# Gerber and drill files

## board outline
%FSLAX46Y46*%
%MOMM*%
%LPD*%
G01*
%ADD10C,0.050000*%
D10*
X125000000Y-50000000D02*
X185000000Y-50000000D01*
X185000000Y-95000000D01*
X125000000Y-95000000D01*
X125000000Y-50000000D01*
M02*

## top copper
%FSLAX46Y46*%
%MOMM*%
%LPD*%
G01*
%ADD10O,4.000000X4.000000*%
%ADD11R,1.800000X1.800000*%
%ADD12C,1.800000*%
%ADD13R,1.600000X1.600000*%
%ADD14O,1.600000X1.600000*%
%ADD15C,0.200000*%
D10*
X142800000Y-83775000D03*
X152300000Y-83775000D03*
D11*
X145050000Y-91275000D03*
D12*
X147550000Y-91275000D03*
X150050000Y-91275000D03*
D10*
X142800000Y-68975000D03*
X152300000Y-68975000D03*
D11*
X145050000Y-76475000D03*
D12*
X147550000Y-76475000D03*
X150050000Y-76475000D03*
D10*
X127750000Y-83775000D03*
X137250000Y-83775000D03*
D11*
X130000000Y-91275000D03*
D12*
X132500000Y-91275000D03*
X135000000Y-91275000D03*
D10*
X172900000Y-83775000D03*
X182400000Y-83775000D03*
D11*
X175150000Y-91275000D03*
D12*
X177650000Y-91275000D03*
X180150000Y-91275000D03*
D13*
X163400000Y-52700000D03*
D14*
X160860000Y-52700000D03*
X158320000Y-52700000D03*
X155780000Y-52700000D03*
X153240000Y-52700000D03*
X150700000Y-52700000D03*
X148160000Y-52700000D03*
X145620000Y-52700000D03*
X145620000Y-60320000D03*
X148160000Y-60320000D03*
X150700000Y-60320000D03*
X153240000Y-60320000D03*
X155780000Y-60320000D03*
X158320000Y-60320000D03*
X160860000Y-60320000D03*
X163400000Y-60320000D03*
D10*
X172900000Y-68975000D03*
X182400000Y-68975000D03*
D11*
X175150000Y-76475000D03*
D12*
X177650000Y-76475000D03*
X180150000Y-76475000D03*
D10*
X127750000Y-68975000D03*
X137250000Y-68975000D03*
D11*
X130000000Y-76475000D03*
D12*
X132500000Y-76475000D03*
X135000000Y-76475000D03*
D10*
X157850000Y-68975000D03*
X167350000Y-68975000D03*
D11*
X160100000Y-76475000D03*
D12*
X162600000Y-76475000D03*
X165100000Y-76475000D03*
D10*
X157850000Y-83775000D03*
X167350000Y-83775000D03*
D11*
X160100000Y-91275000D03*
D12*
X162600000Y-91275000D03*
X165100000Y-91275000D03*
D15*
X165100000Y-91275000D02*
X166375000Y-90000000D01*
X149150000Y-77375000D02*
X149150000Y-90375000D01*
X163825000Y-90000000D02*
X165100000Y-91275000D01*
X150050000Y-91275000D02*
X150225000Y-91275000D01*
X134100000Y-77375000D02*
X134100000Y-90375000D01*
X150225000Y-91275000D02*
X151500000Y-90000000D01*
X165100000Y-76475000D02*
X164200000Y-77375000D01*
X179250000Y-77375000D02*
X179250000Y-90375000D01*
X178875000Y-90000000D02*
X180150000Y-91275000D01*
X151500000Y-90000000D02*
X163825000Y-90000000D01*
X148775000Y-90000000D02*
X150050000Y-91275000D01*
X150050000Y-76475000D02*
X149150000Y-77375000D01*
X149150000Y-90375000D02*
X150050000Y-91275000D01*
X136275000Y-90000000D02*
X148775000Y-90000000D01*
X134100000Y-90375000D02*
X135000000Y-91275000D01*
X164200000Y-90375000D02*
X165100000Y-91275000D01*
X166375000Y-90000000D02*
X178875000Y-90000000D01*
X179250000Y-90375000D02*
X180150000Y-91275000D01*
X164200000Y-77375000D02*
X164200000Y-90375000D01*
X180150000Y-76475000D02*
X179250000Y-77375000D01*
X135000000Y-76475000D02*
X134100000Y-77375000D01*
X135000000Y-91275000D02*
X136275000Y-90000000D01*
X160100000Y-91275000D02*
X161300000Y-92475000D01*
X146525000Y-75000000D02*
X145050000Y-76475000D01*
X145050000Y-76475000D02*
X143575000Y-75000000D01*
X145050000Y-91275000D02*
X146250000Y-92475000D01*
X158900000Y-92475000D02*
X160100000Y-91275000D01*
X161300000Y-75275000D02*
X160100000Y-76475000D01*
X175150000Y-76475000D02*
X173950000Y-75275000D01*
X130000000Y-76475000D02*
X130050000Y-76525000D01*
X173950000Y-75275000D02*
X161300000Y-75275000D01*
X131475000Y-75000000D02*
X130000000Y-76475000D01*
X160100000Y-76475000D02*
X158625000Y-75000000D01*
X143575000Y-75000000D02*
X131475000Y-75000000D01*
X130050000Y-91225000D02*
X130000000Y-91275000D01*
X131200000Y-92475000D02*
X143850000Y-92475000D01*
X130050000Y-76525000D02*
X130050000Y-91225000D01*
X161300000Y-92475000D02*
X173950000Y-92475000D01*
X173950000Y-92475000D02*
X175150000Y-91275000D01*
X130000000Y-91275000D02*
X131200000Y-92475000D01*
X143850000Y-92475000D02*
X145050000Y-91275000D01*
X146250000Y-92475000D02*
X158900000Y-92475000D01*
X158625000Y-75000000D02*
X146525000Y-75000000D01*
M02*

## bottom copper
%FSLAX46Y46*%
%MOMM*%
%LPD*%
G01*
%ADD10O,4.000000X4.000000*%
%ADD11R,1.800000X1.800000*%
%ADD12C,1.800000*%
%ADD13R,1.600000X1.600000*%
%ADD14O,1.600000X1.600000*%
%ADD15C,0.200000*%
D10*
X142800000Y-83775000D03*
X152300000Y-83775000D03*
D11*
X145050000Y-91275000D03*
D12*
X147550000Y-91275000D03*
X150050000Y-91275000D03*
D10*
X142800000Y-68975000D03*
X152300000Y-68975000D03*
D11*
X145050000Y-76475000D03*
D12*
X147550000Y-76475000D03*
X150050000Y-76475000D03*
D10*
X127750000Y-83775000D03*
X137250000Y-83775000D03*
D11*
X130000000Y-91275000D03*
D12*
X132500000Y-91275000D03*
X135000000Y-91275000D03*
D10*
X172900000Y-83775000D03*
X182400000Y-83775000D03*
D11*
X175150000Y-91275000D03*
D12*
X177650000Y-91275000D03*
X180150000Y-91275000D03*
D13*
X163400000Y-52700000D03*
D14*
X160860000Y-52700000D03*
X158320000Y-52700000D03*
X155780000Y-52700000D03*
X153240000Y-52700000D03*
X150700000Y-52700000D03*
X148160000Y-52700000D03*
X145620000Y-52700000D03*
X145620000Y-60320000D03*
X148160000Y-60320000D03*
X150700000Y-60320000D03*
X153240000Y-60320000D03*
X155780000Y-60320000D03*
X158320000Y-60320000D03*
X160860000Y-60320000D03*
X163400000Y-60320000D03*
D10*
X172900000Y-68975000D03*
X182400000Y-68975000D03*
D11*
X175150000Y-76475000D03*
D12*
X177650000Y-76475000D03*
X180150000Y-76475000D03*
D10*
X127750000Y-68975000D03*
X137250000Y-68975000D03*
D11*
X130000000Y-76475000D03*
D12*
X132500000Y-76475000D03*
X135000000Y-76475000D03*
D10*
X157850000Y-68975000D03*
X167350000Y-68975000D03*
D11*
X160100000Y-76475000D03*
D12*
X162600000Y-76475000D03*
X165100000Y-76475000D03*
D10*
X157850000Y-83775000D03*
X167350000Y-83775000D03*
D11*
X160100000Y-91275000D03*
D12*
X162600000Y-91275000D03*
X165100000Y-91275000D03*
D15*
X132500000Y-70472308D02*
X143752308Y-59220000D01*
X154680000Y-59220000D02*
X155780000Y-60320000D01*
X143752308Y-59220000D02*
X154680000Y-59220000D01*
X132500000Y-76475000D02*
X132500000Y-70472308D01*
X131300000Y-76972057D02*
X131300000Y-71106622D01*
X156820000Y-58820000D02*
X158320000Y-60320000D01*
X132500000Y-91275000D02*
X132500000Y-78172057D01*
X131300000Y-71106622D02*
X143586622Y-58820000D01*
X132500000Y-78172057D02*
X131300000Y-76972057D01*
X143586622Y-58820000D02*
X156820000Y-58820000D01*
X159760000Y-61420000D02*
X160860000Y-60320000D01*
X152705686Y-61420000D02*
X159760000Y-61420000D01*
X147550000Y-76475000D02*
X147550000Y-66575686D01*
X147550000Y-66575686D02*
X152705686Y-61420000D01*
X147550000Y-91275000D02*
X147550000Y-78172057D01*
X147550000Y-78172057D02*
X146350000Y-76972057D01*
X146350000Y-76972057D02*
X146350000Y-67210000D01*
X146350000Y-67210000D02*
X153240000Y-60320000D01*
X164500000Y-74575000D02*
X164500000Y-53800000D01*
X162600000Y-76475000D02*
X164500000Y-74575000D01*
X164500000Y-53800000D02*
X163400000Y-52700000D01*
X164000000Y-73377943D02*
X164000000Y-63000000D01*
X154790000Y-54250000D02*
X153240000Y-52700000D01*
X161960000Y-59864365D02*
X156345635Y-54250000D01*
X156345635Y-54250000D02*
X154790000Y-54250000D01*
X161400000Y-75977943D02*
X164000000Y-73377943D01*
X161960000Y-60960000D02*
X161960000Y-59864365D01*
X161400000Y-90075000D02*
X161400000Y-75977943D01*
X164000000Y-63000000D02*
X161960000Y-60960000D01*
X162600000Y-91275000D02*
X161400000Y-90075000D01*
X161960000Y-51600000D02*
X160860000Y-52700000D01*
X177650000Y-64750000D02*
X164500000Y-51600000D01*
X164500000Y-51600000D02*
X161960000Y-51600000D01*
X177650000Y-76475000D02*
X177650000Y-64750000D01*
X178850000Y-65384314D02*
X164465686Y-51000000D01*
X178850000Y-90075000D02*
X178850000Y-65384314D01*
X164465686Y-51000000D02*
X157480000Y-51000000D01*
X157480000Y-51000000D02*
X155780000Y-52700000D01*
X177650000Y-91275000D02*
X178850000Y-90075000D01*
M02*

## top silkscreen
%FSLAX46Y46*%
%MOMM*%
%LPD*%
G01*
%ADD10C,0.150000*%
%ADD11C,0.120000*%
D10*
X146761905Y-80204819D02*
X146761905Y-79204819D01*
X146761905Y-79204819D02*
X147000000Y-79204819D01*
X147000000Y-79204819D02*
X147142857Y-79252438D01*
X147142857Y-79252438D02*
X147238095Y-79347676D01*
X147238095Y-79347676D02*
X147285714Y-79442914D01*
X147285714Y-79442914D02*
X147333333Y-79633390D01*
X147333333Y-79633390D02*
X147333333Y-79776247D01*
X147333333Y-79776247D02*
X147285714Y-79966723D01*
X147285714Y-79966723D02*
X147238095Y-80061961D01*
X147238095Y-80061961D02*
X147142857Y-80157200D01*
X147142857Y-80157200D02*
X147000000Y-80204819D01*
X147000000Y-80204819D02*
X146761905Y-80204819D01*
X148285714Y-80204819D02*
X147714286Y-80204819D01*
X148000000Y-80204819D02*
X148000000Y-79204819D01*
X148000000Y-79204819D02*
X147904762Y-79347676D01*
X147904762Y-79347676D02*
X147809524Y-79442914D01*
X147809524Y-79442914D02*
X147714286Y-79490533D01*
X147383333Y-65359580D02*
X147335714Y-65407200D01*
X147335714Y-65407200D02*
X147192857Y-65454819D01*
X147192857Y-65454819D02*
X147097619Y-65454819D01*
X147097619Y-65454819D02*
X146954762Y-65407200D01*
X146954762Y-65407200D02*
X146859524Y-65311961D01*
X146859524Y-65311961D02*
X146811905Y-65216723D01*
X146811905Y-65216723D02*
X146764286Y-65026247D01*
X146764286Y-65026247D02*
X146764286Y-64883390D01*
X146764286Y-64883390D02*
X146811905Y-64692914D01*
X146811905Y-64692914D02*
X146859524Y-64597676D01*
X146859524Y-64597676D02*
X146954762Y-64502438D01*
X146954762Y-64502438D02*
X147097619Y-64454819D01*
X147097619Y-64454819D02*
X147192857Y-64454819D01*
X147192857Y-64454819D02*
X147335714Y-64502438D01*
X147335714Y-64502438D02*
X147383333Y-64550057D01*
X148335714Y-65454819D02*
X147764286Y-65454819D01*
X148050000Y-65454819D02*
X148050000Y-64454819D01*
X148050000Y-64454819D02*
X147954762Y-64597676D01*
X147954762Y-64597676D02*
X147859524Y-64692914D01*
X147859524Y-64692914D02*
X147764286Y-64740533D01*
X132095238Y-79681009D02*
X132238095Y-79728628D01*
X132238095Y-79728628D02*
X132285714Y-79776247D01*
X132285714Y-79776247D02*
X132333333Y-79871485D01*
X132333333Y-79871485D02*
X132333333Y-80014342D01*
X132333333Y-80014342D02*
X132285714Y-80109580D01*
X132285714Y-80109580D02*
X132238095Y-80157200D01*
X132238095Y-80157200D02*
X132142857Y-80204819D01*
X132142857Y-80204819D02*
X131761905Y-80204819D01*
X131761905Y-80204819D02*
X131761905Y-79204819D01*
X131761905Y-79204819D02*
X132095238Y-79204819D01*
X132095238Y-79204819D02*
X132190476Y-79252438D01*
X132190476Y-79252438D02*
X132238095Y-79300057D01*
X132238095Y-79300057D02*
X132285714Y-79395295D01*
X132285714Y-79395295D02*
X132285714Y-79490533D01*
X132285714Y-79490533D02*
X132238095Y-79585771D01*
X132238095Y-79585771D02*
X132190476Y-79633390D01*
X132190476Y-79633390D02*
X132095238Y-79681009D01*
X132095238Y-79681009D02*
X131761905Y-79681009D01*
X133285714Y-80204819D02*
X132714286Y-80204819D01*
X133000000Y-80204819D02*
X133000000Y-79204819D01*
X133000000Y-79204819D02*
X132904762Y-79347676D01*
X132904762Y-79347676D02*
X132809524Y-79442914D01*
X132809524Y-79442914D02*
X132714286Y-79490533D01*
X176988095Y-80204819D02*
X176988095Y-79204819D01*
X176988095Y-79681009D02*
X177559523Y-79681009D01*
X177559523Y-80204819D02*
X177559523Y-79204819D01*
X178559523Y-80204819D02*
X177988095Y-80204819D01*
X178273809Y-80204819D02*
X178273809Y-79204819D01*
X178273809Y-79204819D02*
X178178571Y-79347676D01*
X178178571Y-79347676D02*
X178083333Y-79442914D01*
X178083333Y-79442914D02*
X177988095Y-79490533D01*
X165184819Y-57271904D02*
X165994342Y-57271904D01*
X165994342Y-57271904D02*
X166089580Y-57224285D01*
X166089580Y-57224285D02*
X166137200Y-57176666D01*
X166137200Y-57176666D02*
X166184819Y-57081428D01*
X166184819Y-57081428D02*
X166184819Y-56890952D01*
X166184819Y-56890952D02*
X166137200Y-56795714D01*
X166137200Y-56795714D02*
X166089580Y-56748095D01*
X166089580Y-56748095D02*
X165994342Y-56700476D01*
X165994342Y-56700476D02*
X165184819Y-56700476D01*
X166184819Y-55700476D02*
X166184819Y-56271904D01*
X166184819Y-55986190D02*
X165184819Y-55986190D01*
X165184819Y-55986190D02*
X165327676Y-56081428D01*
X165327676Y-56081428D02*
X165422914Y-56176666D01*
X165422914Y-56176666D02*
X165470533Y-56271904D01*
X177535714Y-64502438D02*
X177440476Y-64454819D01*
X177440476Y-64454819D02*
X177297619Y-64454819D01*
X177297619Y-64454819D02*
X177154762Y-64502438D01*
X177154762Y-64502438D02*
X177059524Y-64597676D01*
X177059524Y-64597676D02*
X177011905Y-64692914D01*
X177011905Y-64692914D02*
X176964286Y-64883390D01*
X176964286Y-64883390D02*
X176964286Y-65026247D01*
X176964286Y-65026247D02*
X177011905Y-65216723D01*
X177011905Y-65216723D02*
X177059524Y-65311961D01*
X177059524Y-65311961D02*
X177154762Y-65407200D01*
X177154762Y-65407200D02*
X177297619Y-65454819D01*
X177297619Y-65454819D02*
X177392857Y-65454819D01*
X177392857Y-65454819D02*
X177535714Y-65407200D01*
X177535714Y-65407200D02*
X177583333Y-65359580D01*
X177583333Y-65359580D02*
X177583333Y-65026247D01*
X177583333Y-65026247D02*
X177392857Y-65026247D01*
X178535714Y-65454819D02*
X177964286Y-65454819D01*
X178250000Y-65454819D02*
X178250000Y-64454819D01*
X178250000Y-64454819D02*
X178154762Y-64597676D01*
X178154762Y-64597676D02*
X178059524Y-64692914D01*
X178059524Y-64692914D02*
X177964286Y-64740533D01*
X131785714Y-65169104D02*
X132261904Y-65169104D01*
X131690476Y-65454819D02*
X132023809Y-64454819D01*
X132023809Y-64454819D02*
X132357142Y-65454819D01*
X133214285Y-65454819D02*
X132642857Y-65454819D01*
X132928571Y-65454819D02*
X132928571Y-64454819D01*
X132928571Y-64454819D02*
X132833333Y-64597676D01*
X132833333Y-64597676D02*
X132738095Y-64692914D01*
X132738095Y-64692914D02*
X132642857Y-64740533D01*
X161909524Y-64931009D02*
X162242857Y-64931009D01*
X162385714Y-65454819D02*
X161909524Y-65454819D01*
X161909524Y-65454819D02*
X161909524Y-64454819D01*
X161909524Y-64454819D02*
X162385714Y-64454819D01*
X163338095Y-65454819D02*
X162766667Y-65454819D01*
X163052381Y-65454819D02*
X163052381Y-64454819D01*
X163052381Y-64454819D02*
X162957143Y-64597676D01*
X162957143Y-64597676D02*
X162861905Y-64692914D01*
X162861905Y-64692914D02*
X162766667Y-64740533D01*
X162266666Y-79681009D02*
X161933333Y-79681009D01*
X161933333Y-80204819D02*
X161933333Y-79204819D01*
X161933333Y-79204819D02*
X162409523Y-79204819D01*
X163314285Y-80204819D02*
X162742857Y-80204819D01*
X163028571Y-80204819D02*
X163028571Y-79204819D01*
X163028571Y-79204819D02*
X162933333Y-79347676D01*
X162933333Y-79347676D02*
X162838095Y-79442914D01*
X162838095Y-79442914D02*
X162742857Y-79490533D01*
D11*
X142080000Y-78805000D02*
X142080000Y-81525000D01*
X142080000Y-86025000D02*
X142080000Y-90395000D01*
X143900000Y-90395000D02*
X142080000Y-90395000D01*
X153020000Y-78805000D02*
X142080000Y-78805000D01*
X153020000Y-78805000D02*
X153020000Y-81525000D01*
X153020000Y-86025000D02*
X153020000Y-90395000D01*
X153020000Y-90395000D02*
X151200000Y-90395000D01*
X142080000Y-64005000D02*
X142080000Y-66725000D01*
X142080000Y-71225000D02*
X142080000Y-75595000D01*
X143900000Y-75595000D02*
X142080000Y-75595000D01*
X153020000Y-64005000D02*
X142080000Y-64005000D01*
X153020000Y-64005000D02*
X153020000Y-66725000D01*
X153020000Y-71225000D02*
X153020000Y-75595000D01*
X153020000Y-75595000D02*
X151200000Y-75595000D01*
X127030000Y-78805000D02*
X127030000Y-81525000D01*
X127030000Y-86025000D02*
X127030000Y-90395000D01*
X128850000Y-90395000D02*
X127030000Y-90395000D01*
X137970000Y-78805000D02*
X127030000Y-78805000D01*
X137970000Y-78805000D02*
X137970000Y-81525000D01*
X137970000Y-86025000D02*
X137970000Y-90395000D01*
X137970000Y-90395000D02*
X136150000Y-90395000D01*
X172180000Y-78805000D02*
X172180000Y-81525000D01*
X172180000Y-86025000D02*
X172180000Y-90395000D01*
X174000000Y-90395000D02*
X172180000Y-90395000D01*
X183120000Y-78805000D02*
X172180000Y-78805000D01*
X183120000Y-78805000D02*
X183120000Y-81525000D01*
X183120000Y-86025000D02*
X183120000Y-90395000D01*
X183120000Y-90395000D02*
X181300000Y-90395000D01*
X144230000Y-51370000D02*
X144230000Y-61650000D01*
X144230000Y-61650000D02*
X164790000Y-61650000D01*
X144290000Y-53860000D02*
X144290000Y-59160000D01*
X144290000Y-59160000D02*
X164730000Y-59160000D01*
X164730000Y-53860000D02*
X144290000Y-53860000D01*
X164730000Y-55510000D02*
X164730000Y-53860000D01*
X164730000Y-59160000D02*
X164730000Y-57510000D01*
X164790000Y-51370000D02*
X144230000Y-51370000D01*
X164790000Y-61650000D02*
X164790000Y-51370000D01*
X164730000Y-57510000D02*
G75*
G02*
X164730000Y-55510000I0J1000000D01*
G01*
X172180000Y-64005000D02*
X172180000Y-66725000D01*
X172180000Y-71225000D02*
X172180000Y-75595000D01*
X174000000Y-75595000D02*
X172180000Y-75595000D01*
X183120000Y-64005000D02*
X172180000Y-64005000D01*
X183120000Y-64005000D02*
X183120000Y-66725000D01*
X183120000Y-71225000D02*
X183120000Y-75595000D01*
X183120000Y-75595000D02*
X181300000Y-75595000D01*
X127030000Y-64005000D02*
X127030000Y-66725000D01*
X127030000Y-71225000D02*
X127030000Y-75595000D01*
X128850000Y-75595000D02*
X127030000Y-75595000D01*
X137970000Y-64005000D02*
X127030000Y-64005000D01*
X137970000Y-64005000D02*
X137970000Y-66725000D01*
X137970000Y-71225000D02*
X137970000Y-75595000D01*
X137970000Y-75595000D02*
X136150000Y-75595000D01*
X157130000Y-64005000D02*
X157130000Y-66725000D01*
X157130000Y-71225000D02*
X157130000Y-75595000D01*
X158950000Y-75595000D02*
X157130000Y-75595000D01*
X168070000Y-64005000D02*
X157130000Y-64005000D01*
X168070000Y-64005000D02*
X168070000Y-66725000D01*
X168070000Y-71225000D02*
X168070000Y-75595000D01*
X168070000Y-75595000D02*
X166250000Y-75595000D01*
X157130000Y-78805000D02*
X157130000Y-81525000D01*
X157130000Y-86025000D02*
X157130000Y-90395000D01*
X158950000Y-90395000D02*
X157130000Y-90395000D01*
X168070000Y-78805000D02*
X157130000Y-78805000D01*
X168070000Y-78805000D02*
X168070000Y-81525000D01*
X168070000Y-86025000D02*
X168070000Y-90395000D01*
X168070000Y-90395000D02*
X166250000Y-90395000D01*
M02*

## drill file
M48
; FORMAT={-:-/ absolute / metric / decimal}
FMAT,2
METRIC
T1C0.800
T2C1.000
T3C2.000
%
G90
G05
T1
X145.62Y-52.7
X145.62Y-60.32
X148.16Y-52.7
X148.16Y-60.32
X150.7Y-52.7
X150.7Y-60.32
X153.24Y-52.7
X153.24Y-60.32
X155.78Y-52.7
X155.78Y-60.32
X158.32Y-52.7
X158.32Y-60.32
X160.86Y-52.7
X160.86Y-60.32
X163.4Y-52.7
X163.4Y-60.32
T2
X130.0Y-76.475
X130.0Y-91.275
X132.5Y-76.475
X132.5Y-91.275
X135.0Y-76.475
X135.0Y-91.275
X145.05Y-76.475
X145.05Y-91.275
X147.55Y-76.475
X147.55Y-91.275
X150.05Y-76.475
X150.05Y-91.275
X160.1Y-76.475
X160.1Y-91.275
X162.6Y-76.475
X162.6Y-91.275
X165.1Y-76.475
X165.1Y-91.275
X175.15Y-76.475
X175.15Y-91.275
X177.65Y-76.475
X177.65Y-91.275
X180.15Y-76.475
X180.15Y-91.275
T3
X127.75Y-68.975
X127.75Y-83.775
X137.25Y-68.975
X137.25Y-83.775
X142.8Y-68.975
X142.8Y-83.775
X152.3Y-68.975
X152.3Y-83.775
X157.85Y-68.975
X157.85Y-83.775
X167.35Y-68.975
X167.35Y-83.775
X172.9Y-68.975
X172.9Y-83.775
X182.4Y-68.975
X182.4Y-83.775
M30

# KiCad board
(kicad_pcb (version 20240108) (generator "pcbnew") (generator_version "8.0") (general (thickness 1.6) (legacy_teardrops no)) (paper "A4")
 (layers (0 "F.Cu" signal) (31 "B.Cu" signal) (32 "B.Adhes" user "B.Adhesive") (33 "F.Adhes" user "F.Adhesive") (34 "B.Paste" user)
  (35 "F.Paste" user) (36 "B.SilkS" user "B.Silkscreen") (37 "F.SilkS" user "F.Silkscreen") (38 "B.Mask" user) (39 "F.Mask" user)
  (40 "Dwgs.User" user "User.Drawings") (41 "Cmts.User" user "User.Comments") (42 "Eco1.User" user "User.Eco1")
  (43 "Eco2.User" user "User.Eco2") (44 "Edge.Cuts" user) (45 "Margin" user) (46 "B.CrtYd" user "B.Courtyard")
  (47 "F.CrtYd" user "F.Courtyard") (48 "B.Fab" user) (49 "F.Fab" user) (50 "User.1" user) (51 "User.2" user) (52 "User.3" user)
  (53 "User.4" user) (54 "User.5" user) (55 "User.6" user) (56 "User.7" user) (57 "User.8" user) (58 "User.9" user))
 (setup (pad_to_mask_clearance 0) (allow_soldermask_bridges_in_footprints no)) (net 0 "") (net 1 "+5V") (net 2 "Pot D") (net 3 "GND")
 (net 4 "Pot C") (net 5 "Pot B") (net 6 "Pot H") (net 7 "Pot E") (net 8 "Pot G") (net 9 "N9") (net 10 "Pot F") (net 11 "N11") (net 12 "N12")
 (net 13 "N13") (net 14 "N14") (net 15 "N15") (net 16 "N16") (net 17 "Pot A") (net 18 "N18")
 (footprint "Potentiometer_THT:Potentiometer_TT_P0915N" (layer "F.Cu") (at 145.05 91.275)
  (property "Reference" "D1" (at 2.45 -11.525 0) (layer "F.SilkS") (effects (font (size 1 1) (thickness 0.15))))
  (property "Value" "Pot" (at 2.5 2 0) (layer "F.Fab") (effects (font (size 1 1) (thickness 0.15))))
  (fp_line (start -2.97 -12.47) (end -2.97 -9.75) (stroke (width 0.12) (type solid)) (layer "F.SilkS"))
  (fp_line (start -2.97 -5.25) (end -2.97 -0.88) (stroke (width 0.12) (type solid)) (layer "F.SilkS"))
  (fp_line (start -1.15 -0.88) (end -2.97 -0.88) (stroke (width 0.12) (type solid)) (layer "F.SilkS"))
  (fp_line (start 7.97 -12.47) (end -2.97 -12.47) (stroke (width 0.12) (type solid)) (layer "F.SilkS"))
  (fp_line (start 7.97 -12.47) (end 7.97 -9.75) (stroke (width 0.12) (type solid)) (layer "F.SilkS"))
  (fp_line (start 7.97 -5.25) (end 7.97 -0.88) (stroke (width 0.12) (type solid)) (layer "F.SilkS"))
  (fp_line (start 7.97 -0.88) (end 6.15 -0.88) (stroke (width 0.12) (type solid)) (layer "F.SilkS"))
  (pad "" thru_hole oval (at -2.25 -7.5) (size 4 4) (drill 2) (layers "*.Cu" "*.Mask") (remove_unused_layers no))
  (pad "" thru_hole oval (at 7.25 -7.5) (size 4 4) (drill 2) (layers "*.Cu" "*.Mask") (remove_unused_layers no))
  (pad "1" thru_hole rect (at 0 0) (size 1.8 1.8) (drill 1) (layers "*.Cu" "*.Mask") (remove_unused_layers no) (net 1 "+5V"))
  (pad "2" thru_hole circle (at 2.5 0) (size 1.8 1.8) (drill 1) (layers "*.Cu" "*.Mask") (remove_unused_layers no) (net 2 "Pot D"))
  (pad "3" thru_hole circle (at 5 0) (size 1.8 1.8) (drill 1) (layers "*.Cu" "*.Mask") (remove_unused_layers no) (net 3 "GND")))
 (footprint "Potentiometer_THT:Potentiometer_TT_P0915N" (layer "F.Cu") (at 145.05 76.475)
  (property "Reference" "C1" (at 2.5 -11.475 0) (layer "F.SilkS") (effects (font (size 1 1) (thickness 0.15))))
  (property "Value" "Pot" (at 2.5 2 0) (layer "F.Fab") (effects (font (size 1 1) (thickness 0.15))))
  (fp_line (start -2.97 -12.47) (end -2.97 -9.75) (stroke (width 0.12) (type solid)) (layer "F.SilkS"))
  (fp_line (start -2.97 -5.25) (end -2.97 -0.88) (stroke (width 0.12) (type solid)) (layer "F.SilkS"))
  (fp_line (start -1.15 -0.88) (end -2.97 -0.88) (stroke (width 0.12) (type solid)) (layer "F.SilkS"))
  (fp_line (start 7.97 -12.47) (end -2.97 -12.47) (stroke (width 0.12) (type solid)) (layer "F.SilkS"))
  (fp_line (start 7.97 -12.47) (end 7.97 -9.75) (stroke (width 0.12) (type solid)) (layer "F.SilkS"))
  (fp_line (start 7.97 -5.25) (end 7.97 -0.88) (stroke (width 0.12) (type solid)) (layer "F.SilkS"))
  (fp_line (start 7.97 -0.88) (end 6.15 -0.88) (stroke (width 0.12) (type solid)) (layer "F.SilkS"))
  (pad "" thru_hole oval (at -2.25 -7.5) (size 4 4) (drill 2) (layers "*.Cu" "*.Mask") (remove_unused_layers no))
  (pad "" thru_hole oval (at 7.25 -7.5) (size 4 4) (drill 2) (layers "*.Cu" "*.Mask") (remove_unused_layers no))
  (pad "1" thru_hole rect (at 0 0) (size 1.8 1.8) (drill 1) (layers "*.Cu" "*.Mask") (remove_unused_layers no) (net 1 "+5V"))
  (pad "2" thru_hole circle (at 2.5 0) (size 1.8 1.8) (drill 1) (layers "*.Cu" "*.Mask") (remove_unused_layers no) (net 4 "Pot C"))
  (pad "3" thru_hole circle (at 5 0) (size 1.8 1.8) (drill 1) (layers "*.Cu" "*.Mask") (remove_unused_layers no) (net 3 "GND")))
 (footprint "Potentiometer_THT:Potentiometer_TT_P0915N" (layer "F.Cu") (at 130 91.275)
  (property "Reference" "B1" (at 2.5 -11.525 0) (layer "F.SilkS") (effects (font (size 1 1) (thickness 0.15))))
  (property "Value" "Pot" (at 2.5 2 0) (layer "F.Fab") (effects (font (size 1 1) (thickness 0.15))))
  (fp_line (start -2.97 -12.47) (end -2.97 -9.75) (stroke (width 0.12) (type solid)) (layer "F.SilkS"))
  (fp_line (start -2.97 -5.25) (end -2.97 -0.88) (stroke (width 0.12) (type solid)) (layer "F.SilkS"))
  (fp_line (start -1.15 -0.88) (end -2.97 -0.88) (stroke (width 0.12) (type solid)) (layer "F.SilkS"))
  (fp_line (start 7.97 -12.47) (end -2.97 -12.47) (stroke (width 0.12) (type solid)) (layer "F.SilkS"))
  (fp_line (start 7.97 -12.47) (end 7.97 -9.75) (stroke (width 0.12) (type solid)) (layer "F.SilkS"))
  (fp_line (start 7.97 -5.25) (end 7.97 -0.88) (stroke (width 0.12) (type solid)) (layer "F.SilkS"))
  (fp_line (start 7.97 -0.88) (end 6.15 -0.88) (stroke (width 0.12) (type solid)) (layer "F.SilkS"))
  (pad "" thru_hole oval (at -2.25 -7.5) (size 4 4) (drill 2) (layers "*.Cu" "*.Mask") (remove_unused_layers no))
  (pad "" thru_hole oval (at 7.25 -7.5) (size 4 4) (drill 2) (layers "*.Cu" "*.Mask") (remove_unused_layers no))
  (pad "1" thru_hole rect (at 0 0) (size 1.8 1.8) (drill 1) (layers "*.Cu" "*.Mask") (remove_unused_layers no) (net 1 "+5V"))
  (pad "2" thru_hole circle (at 2.5 0) (size 1.8 1.8) (drill 1) (layers "*.Cu" "*.Mask") (remove_unused_layers no) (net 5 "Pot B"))
  (pad "3" thru_hole circle (at 5 0) (size 1.8 1.8) (drill 1) (layers "*.Cu" "*.Mask") (remove_unused_layers no) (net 3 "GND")))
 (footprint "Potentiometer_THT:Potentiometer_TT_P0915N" (layer "F.Cu") (at 175.15 91.275)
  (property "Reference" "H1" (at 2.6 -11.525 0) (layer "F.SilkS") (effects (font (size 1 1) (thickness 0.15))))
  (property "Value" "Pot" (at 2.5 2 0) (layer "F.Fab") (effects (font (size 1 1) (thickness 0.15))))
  (fp_line (start -2.97 -12.47) (end -2.97 -9.75) (stroke (width 0.12) (type solid)) (layer "F.SilkS"))
  (fp_line (start -2.97 -5.25) (end -2.97 -0.88) (stroke (width 0.12) (type solid)) (layer "F.SilkS"))
  (fp_line (start -1.15 -0.88) (end -2.97 -0.88) (stroke (width 0.12) (type solid)) (layer "F.SilkS"))
  (fp_line (start 7.97 -12.47) (end -2.97 -12.47) (stroke (width 0.12) (type solid)) (layer "F.SilkS"))
  (fp_line (start 7.97 -12.47) (end 7.97 -9.75) (stroke (width 0.12) (type solid)) (layer "F.SilkS"))
  (fp_line (start 7.97 -5.25) (end 7.97 -0.88) (stroke (width 0.12) (type solid)) (layer "F.SilkS"))
  (fp_line (start 7.97 -0.88) (end 6.15 -0.88) (stroke (width 0.12) (type solid)) (layer "F.SilkS"))
  (pad "" thru_hole oval (at -2.25 -7.5) (size 4 4) (drill 2) (layers "*.Cu" "*.Mask") (remove_unused_layers no))
  (pad "" thru_hole oval (at 7.25 -7.5) (size 4 4) (drill 2) (layers "*.Cu" "*.Mask") (remove_unused_layers no))
  (pad "1" thru_hole rect (at 0 0) (size 1.8 1.8) (drill 1) (layers "*.Cu" "*.Mask") (remove_unused_layers no) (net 1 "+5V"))
  (pad "2" thru_hole circle (at 2.5 0) (size 1.8 1.8) (drill 1) (layers "*.Cu" "*.Mask") (remove_unused_layers no) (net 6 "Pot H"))
  (pad "3" thru_hole circle (at 5 0) (size 1.8 1.8) (drill 1) (layers "*.Cu" "*.Mask") (remove_unused_layers no) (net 3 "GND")))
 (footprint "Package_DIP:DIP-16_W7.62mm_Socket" (layer "F.Cu") (at 163.4 52.7 -90)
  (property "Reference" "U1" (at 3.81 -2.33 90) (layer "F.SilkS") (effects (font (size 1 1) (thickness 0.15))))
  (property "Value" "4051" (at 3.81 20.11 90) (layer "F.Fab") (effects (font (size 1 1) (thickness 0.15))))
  (fp_line (start -1.33 19.17) (end 8.95 19.17) (stroke (width 0.12) (type solid)) (layer "F.SilkS"))
  (fp_line (start 8.95 19.17) (end 8.95 -1.39) (stroke (width 0.12) (type solid)) (layer "F.SilkS"))
  (fp_line (start 1.16 19.11) (end 6.46 19.11) (stroke (width 0.12) (type solid)) (layer "F.SilkS"))
  (fp_line (start 6.46 19.11) (end 6.46 -1.33) (stroke (width 0.12) (type solid)) (layer "F.SilkS"))
  (fp_line (start 1.16 -1.33) (end 1.16 19.11) (stroke (width 0.12) (type solid)) (layer "F.SilkS"))
  (fp_line (start 2.81 -1.33) (end 1.16 -1.33) (stroke (width 0.12) (type solid)) (layer "F.SilkS"))
  (fp_line (start 6.46 -1.33) (end 4.81 -1.33) (stroke (width 0.12) (type solid)) (layer "F.SilkS"))
  (fp_line (start -1.33 -1.39) (end -1.33 19.17) (stroke (width 0.12) (type solid)) (layer "F.SilkS"))
  (fp_line (start 8.95 -1.39) (end -1.33 -1.39) (stroke (width 0.12) (type solid)) (layer "F.SilkS"))
  (fp_arc (start 4.81 -1.33) (mid 3.81 -0.33) (end 2.81 -1.33) (stroke (width 0.12) (type solid)) (layer "F.SilkS"))
  (pad "1" thru_hole rect (at 0 0 270) (size 1.6 1.6) (drill 0.8) (layers "*.Cu" "*.Mask") (remove_unused_layers no) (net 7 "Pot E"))
  (pad "2" thru_hole oval (at 0 2.54 270) (size 1.6 1.6) (drill 0.8) (layers "*.Cu" "*.Mask") (remove_unused_layers no) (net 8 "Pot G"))
  (pad "3" thru_hole oval (at 0 5.08 270) (size 1.6 1.6) (drill 0.8) (layers "*.Cu" "*.Mask") (remove_unused_layers no) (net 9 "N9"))
  (pad "4" thru_hole oval (at 0 7.62 270) (size 1.6 1.6) (drill 0.8) (layers "*.Cu" "*.Mask") (remove_unused_layers no) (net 6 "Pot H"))
  (pad "5" thru_hole oval (at 0 10.16 270) (size 1.6 1.6) (drill 0.8) (layers "*.Cu" "*.Mask") (remove_unused_layers no) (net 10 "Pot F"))
  (pad "6" thru_hole oval (at 0 12.7 270) (size 1.6 1.6) (drill 0.8) (layers "*.Cu" "*.Mask") (remove_unused_layers no) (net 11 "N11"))
  (pad "7" thru_hole oval (at 0 15.24 270) (size 1.6 1.6) (drill 0.8) (layers "*.Cu" "*.Mask") (remove_unused_layers no) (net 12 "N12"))
  (pad "8" thru_hole oval (at 0 17.78 270) (size 1.6 1.6) (drill 0.8) (layers "*.Cu" "*.Mask") (remove_unused_layers no) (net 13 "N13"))
  (pad "9" thru_hole oval (at 7.62 17.78 270) (size 1.6 1.6) (drill 0.8) (layers "*.Cu" "*.Mask") (remove_unused_layers no) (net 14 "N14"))
  (pad "10" thru_hole oval (at 7.62 15.24 270) (size 1.6 1.6) (drill 0.8) (layers "*.Cu" "*.Mask") (remove_unused_layers no) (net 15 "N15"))
  (pad "11" thru_hole oval (at 7.62 12.7 270) (size 1.6 1.6) (drill 0.8) (layers "*.Cu" "*.Mask") (remove_unused_layers no) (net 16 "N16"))
  (pad "12" thru_hole oval (at 7.62 10.16 270) (size 1.6 1.6) (drill 0.8) (layers "*.Cu" "*.Mask") (remove_unused_layers no) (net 2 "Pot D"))
  (pad "13" thru_hole oval (at 7.62 7.62 270) (size 1.6 1.6) (drill 0.8) (layers "*.Cu" "*.Mask") (remove_unused_layers no) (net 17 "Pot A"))
  (pad "14" thru_hole oval (at 7.62 5.08 270) (size 1.6 1.6) (drill 0.8) (layers "*.Cu" "*.Mask") (remove_unused_layers no) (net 5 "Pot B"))
  (pad "15" thru_hole oval (at 7.62 2.54 270) (size 1.6 1.6) (drill 0.8) (layers "*.Cu" "*.Mask") (remove_unused_layers no) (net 4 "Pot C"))
  (pad "16" thru_hole oval (at 7.62 0 270) (size 1.6 1.6) (drill 0.8) (layers "*.Cu" "*.Mask") (remove_unused_layers no) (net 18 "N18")))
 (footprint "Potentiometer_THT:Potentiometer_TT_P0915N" (layer "F.Cu") (at 175.15 76.475)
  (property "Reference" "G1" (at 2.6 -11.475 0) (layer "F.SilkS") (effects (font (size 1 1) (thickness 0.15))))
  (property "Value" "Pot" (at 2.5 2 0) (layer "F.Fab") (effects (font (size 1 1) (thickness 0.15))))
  (fp_line (start -2.97 -12.47) (end -2.97 -9.75) (stroke (width 0.12) (type solid)) (layer "F.SilkS"))
  (fp_line (start -2.97 -5.25) (end -2.97 -0.88) (stroke (width 0.12) (type solid)) (layer "F.SilkS"))
  (fp_line (start -1.15 -0.88) (end -2.97 -0.88) (stroke (width 0.12) (type solid)) (layer "F.SilkS"))
  (fp_line (start 7.97 -12.47) (end -2.97 -12.47) (stroke (width 0.12) (type solid)) (layer "F.SilkS"))
  (fp_line (start 7.97 -12.47) (end 7.97 -9.75) (stroke (width 0.12) (type solid)) (layer "F.SilkS"))
  (fp_line (start 7.97 -5.25) (end 7.97 -0.88) (stroke (width 0.12) (type solid)) (layer "F.SilkS"))
  (fp_line (start 7.97 -0.88) (end 6.15 -0.88) (stroke (width 0.12) (type solid)) (layer "F.SilkS"))
  (pad "" thru_hole oval (at -2.25 -7.5) (size 4 4) (drill 2) (layers "*.Cu" "*.Mask") (remove_unused_layers no))
  (pad "" thru_hole oval (at 7.25 -7.5) (size 4 4) (drill 2) (layers "*.Cu" "*.Mask") (remove_unused_layers no))
  (pad "1" thru_hole rect (at 0 0) (size 1.8 1.8) (drill 1) (layers "*.Cu" "*.Mask") (remove_unused_layers no) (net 1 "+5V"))
  (pad "2" thru_hole circle (at 2.5 0) (size 1.8 1.8) (drill 1) (layers "*.Cu" "*.Mask") (remove_unused_layers no) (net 8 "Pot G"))
  (pad "3" thru_hole circle (at 5 0) (size 1.8 1.8) (drill 1) (layers "*.Cu" "*.Mask") (remove_unused_layers no) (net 3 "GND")))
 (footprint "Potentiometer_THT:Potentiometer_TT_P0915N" (layer "F.Cu") (at 130 76.475)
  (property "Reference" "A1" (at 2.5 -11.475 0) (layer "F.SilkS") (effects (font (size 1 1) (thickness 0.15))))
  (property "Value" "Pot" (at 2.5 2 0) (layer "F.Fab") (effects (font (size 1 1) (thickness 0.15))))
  (fp_line (start -2.97 -12.47) (end -2.97 -9.75) (stroke (width 0.12) (type solid)) (layer "F.SilkS"))
  (fp_line (start -2.97 -5.25) (end -2.97 -0.88) (stroke (width 0.12) (type solid)) (layer "F.SilkS"))
  (fp_line (start -1.15 -0.88) (end -2.97 -0.88) (stroke (width 0.12) (type solid)) (layer "F.SilkS"))
  (fp_line (start 7.97 -12.47) (end -2.97 -12.47) (stroke (width 0.12) (type solid)) (layer "F.SilkS"))
  (fp_line (start 7.97 -12.47) (end 7.97 -9.75) (stroke (width 0.12) (type solid)) (layer "F.SilkS"))
  (fp_line (start 7.97 -5.25) (end 7.97 -0.88) (stroke (width 0.12) (type solid)) (layer "F.SilkS"))
  (fp_line (start 7.97 -0.88) (end 6.15 -0.88) (stroke (width 0.12) (type solid)) (layer "F.SilkS"))
  (pad "" thru_hole oval (at -2.25 -7.5) (size 4 4) (drill 2) (layers "*.Cu" "*.Mask") (remove_unused_layers no))
  (pad "" thru_hole oval (at 7.25 -7.5) (size 4 4) (drill 2) (layers "*.Cu" "*.Mask") (remove_unused_layers no))
  (pad "1" thru_hole rect (at 0 0) (size 1.8 1.8) (drill 1) (layers "*.Cu" "*.Mask") (remove_unused_layers no) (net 1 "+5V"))
  (pad "2" thru_hole circle (at 2.5 0) (size 1.8 1.8) (drill 1) (layers "*.Cu" "*.Mask") (remove_unused_layers no) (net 17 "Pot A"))
  (pad "3" thru_hole circle (at 5 0) (size 1.8 1.8) (drill 1) (layers "*.Cu" "*.Mask") (remove_unused_layers no) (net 3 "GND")))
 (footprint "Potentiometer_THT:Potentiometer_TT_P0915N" (layer "F.Cu") (at 160.1 76.475)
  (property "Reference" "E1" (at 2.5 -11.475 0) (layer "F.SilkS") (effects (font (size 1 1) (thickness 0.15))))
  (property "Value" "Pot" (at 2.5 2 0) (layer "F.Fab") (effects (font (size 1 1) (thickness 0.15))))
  (fp_line (start -2.97 -12.47) (end -2.97 -9.75) (stroke (width 0.12) (type solid)) (layer "F.SilkS"))
  (fp_line (start -2.97 -5.25) (end -2.97 -0.88) (stroke (width 0.12) (type solid)) (layer "F.SilkS"))
  (fp_line (start -1.15 -0.88) (end -2.97 -0.88) (stroke (width 0.12) (type solid)) (layer "F.SilkS"))
  (fp_line (start 7.97 -12.47) (end -2.97 -12.47) (stroke (width 0.12) (type solid)) (layer "F.SilkS"))
  (fp_line (start 7.97 -12.47) (end 7.97 -9.75) (stroke (width 0.12) (type solid)) (layer "F.SilkS"))
  (fp_line (start 7.97 -5.25) (end 7.97 -0.88) (stroke (width 0.12) (type solid)) (layer "F.SilkS"))
  (fp_line (start 7.97 -0.88) (end 6.15 -0.88) (stroke (width 0.12) (type solid)) (layer "F.SilkS"))
  (pad "" thru_hole oval (at -2.25 -7.5) (size 4 4) (drill 2) (layers "*.Cu" "*.Mask") (remove_unused_layers no))
  (pad "" thru_hole oval (at 7.25 -7.5) (size 4 4) (drill 2) (layers "*.Cu" "*.Mask") (remove_unused_layers no))
  (pad "1" thru_hole rect (at 0 0) (size 1.8 1.8) (drill 1) (layers "*.Cu" "*.Mask") (remove_unused_layers no) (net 1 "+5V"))
  (pad "2" thru_hole circle (at 2.5 0) (size 1.8 1.8) (drill 1) (layers "*.Cu" "*.Mask") (remove_unused_layers no) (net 7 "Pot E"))
  (pad "3" thru_hole circle (at 5 0) (size 1.8 1.8) (drill 1) (layers "*.Cu" "*.Mask") (remove_unused_layers no) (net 3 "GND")))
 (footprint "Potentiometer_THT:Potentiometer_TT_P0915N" (layer "F.Cu") (at 160.1 91.275)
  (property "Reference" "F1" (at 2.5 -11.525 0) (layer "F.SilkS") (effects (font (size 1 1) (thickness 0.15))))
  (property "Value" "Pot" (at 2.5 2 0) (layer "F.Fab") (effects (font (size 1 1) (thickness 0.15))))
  (fp_line (start -2.97 -12.47) (end -2.97 -9.75) (stroke (width 0.12) (type solid)) (layer "F.SilkS"))
  (fp_line (start -2.97 -5.25) (end -2.97 -0.88) (stroke (width 0.12) (type solid)) (layer "F.SilkS"))
  (fp_line (start -1.15 -0.88) (end -2.97 -0.88) (stroke (width 0.12) (type solid)) (layer "F.SilkS"))
  (fp_line (start 7.97 -12.47) (end -2.97 -12.47) (stroke (width 0.12) (type solid)) (layer "F.SilkS"))
  (fp_line (start 7.97 -12.47) (end 7.97 -9.75) (stroke (width 0.12) (type solid)) (layer "F.SilkS"))
  (fp_line (start 7.97 -5.25) (end 7.97 -0.88) (stroke (width 0.12) (type solid)) (layer "F.SilkS"))
  (fp_line (start 7.97 -0.88) (end 6.15 -0.88) (stroke (width 0.12) (type solid)) (layer "F.SilkS"))
  (pad "" thru_hole oval (at -2.25 -7.5) (size 4 4) (drill 2) (layers "*.Cu" "*.Mask") (remove_unused_layers no))
  (pad "" thru_hole oval (at 7.25 -7.5) (size 4 4) (drill 2) (layers "*.Cu" "*.Mask") (remove_unused_layers no))
  (pad "1" thru_hole rect (at 0 0) (size 1.8 1.8) (drill 1) (layers "*.Cu" "*.Mask") (remove_unused_layers no) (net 1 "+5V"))
  (pad "2" thru_hole circle (at 2.5 0) (size 1.8 1.8) (drill 1) (layers "*.Cu" "*.Mask") (remove_unused_layers no) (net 10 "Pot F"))
  (pad "3" thru_hole circle (at 5 0) (size 1.8 1.8) (drill 1) (layers "*.Cu" "*.Mask") (remove_unused_layers no) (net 3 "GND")))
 (gr_rect (start 125 50) (end 185 95) (stroke (width 0.05) (type default)) (fill none) (layer "Edge.Cuts"))
 (segment (start 132.5 70.472308) (end 143.752308 59.22) (width 0.2) (layer "B.Cu") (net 17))
 (segment (start 154.68 59.22) (end 155.78 60.32) (width 0.2) (layer "B.Cu") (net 17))
 (segment (start 143.752308 59.22) (end 154.68 59.22) (width 0.2) (layer "B.Cu") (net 17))
 (segment (start 132.5 76.475) (end 132.5 70.472308) (width 0.2) (layer "B.Cu") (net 17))
 (segment (start 165.1 91.275) (end 166.375 90) (width 0.2) (layer "F.Cu") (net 3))
 (segment (start 149.15 77.375) (end 149.15 90.375) (width 0.2) (layer "F.Cu") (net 3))
 (segment (start 163.825 90) (end 165.1 91.275) (width 0.2) (layer "F.Cu") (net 3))
 (segment (start 150.05 91.275) (end 150.225 91.275) (width 0.2) (layer "F.Cu") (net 3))
 (segment (start 134.1 77.375) (end 134.1 90.375) (width 0.2) (layer "F.Cu") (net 3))
 (segment (start 150.225 91.275) (end 151.5 90) (width 0.2) (layer "F.Cu") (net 3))
 (segment (start 165.1 76.475) (end 164.2 77.375) (width 0.2) (layer "F.Cu") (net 3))
 (segment (start 179.25 77.375) (end 179.25 90.375) (width 0.2) (layer "F.Cu") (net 3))
 (segment (start 178.875 90) (end 180.15 91.275) (width 0.2) (layer "F.Cu") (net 3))
 (segment (start 151.5 90) (end 163.825 90) (width 0.2) (layer "F.Cu") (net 3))
 (segment (start 148.775 90) (end 150.05 91.275) (width 0.2) (layer "F.Cu") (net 3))
 (segment (start 150.05 76.475) (end 149.15 77.375) (width 0.2) (layer "F.Cu") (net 3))
 (segment (start 149.15 90.375) (end 150.05 91.275) (width 0.2) (layer "F.Cu") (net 3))
 (segment (start 136.275 90) (end 148.775 90) (width 0.2) (layer "F.Cu") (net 3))
 (segment (start 134.1 90.375) (end 135 91.275) (width 0.2) (layer "F.Cu") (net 3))
 (segment (start 164.2 90.375) (end 165.1 91.275) (width 0.2) (layer "F.Cu") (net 3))
 (segment (start 166.375 90) (end 178.875 90) (width 0.2) (layer "F.Cu") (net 3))
 (segment (start 179.25 90.375) (end 180.15 91.275) (width 0.2) (layer "F.Cu") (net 3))
 (segment (start 164.2 77.375) (end 164.2 90.375) (width 0.2) (layer "F.Cu") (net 3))
 (segment (start 180.15 76.475) (end 179.25 77.375) (width 0.2) (layer "F.Cu") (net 3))
 (segment (start 135 76.475) (end 134.1 77.375) (width 0.2) (layer "F.Cu") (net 3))
 (segment (start 135 91.275) (end 136.275 90) (width 0.2) (layer "F.Cu") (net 3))
 (segment (start 160.1 91.275) (end 161.3 92.475) (width 0.2) (layer "F.Cu") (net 1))
 (segment (start 146.525 75) (end 145.05 76.475) (width 0.2) (layer "F.Cu") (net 1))
 (segment (start 145.05 76.475) (end 143.575 75) (width 0.2) (layer "F.Cu") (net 1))
 (segment (start 145.05 91.275) (end 146.25 92.475) (width 0.2) (layer "F.Cu") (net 1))
 (segment (start 158.9 92.475) (end 160.1 91.275) (width 0.2) (layer "F.Cu") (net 1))
 (segment (start 161.3 75.275) (end 160.1 76.475) (width 0.2) (layer "F.Cu") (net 1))
 (segment (start 175.15 76.475) (end 173.95 75.275) (width 0.2) (layer "F.Cu") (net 1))
 (segment (start 130 76.475) (end 130.05 76.525) (width 0.2) (layer "F.Cu") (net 1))
 (segment (start 173.95 75.275) (end 161.3 75.275) (width 0.2) (layer "F.Cu") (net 1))
 (segment (start 131.475 75) (end 130 76.475) (width 0.2) (layer "F.Cu") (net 1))
 (segment (start 160.1 76.475) (end 158.625 75) (width 0.2) (layer "F.Cu") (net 1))
 (segment (start 143.575 75) (end 131.475 75) (width 0.2) (layer "F.Cu") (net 1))
 (segment (start 130.05 91.225) (end 130 91.275) (width 0.2) (layer "F.Cu") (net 1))
 (segment (start 131.2 92.475) (end 143.85 92.475) (width 0.2) (layer "F.Cu") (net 1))
 (segment (start 130.05 76.525) (end 130.05 91.225) (width 0.2) (layer "F.Cu") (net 1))
 (segment (start 161.3 92.475) (end 173.95 92.475) (width 0.2) (layer "F.Cu") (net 1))
 (segment (start 173.95 92.475) (end 175.15 91.275) (width 0.2) (layer "F.Cu") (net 1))
 (segment (start 130 91.275) (end 131.2 92.475) (width 0.2) (layer "F.Cu") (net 1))
 (segment (start 143.85 92.475) (end 145.05 91.275) (width 0.2) (layer "F.Cu") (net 1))
 (segment (start 146.25 92.475) (end 158.9 92.475) (width 0.2) (layer "F.Cu") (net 1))
 (segment (start 158.625 75) (end 146.525 75) (width 0.2) (layer "F.Cu") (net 1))
 (segment (start 131.3 76.972057) (end 131.3 71.106622) (width 0.2) (layer "B.Cu") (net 5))
 (segment (start 156.82 58.82) (end 158.32 60.32) (width 0.2) (layer "B.Cu") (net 5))
 (segment (start 132.5 91.275) (end 132.5 78.172057) (width 0.2) (layer "B.Cu") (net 5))
 (segment (start 131.3 71.106622) (end 143.586622 58.82) (width 0.2) (layer "B.Cu") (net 5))
 (segment (start 132.5 78.172057) (end 131.3 76.972057) (width 0.2) (layer "B.Cu") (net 5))
 (segment (start 143.586622 58.82) (end 156.82 58.82) (width 0.2) (layer "B.Cu") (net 5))
 (segment (start 159.76 61.42) (end 160.86 60.32) (width 0.2) (layer "B.Cu") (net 4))
 (segment (start 152.705686 61.42) (end 159.76 61.42) (width 0.2) (layer "B.Cu") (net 4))
 (segment (start 147.55 76.475) (end 147.55 66.575686) (width 0.2) (layer "B.Cu") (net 4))
 (segment (start 147.55 66.575686) (end 152.705686 61.42) (width 0.2) (layer "B.Cu") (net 4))
 (segment (start 147.55 91.275) (end 147.55 78.172057) (width 0.2) (layer "B.Cu") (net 2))
 (segment (start 147.55 78.172057) (end 146.35 76.972057) (width 0.2) (layer "B.Cu") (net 2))
 (segment (start 146.35 76.972057) (end 146.35 67.21) (width 0.2) (layer "B.Cu") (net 2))
 (segment (start 146.35 67.21) (end 153.24 60.32) (width 0.2) (layer "B.Cu") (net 2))
 (segment (start 164.5 74.575) (end 164.5 53.8) (width 0.2) (layer "B.Cu") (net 7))
 (segment (start 162.6 76.475) (end 164.5 74.575) (width 0.2) (layer "B.Cu") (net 7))
 (segment (start 164.5 53.8) (end 163.4 52.7) (width 0.2) (layer "B.Cu") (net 7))
 (segment (start 164 73.377943) (end 164 63) (width 0.2) (layer "B.Cu") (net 10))
 (segment (start 154.79 54.25) (end 153.24 52.7) (width 0.2) (layer "B.Cu") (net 10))
 (segment (start 161.96 59.864365) (end 156.345635 54.25) (width 0.2) (layer "B.Cu") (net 10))
 (segment (start 156.345635 54.25) (end 154.79 54.25) (width 0.2) (layer "B.Cu") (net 10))
 (segment (start 161.4 75.977943) (end 164 73.377943) (width 0.2) (layer "B.Cu") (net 10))
 (segment (start 161.96 60.96) (end 161.96 59.864365) (width 0.2) (layer "B.Cu") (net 10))
 (segment (start 161.4 90.075) (end 161.4 75.977943) (width 0.2) (layer "B.Cu") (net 10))
 (segment (start 164 63) (end 161.96 60.96) (width 0.2) (layer "B.Cu") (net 10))
 (segment (start 162.6 91.275) (end 161.4 90.075) (width 0.2) (layer "B.Cu") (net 10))
 (segment (start 161.96 51.6) (end 160.86 52.7) (width 0.2) (layer "B.Cu") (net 8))
 (segment (start 177.65 64.75) (end 164.5 51.6) (width 0.2) (layer "B.Cu") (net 8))
 (segment (start 164.5 51.6) (end 161.96 51.6) (width 0.2) (layer "B.Cu") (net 8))
 (segment (start 177.65 76.475) (end 177.65 64.75) (width 0.2) (layer "B.Cu") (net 8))
 (segment (start 178.85 65.384314) (end 164.465686 51) (width 0.2) (layer "B.Cu") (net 6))
 (segment (start 178.85 90.075) (end 178.85 65.384314) (width 0.2) (layer "B.Cu") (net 6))
 (segment (start 164.465686 51) (end 157.48 51) (width 0.2) (layer "B.Cu") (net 6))
 (segment (start 157.48 51) (end 155.78 52.7) (width 0.2) (layer "B.Cu") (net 6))
 (segment (start 177.65 91.275) (end 178.85 90.075) (width 0.2) (layer "B.Cu") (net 6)))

